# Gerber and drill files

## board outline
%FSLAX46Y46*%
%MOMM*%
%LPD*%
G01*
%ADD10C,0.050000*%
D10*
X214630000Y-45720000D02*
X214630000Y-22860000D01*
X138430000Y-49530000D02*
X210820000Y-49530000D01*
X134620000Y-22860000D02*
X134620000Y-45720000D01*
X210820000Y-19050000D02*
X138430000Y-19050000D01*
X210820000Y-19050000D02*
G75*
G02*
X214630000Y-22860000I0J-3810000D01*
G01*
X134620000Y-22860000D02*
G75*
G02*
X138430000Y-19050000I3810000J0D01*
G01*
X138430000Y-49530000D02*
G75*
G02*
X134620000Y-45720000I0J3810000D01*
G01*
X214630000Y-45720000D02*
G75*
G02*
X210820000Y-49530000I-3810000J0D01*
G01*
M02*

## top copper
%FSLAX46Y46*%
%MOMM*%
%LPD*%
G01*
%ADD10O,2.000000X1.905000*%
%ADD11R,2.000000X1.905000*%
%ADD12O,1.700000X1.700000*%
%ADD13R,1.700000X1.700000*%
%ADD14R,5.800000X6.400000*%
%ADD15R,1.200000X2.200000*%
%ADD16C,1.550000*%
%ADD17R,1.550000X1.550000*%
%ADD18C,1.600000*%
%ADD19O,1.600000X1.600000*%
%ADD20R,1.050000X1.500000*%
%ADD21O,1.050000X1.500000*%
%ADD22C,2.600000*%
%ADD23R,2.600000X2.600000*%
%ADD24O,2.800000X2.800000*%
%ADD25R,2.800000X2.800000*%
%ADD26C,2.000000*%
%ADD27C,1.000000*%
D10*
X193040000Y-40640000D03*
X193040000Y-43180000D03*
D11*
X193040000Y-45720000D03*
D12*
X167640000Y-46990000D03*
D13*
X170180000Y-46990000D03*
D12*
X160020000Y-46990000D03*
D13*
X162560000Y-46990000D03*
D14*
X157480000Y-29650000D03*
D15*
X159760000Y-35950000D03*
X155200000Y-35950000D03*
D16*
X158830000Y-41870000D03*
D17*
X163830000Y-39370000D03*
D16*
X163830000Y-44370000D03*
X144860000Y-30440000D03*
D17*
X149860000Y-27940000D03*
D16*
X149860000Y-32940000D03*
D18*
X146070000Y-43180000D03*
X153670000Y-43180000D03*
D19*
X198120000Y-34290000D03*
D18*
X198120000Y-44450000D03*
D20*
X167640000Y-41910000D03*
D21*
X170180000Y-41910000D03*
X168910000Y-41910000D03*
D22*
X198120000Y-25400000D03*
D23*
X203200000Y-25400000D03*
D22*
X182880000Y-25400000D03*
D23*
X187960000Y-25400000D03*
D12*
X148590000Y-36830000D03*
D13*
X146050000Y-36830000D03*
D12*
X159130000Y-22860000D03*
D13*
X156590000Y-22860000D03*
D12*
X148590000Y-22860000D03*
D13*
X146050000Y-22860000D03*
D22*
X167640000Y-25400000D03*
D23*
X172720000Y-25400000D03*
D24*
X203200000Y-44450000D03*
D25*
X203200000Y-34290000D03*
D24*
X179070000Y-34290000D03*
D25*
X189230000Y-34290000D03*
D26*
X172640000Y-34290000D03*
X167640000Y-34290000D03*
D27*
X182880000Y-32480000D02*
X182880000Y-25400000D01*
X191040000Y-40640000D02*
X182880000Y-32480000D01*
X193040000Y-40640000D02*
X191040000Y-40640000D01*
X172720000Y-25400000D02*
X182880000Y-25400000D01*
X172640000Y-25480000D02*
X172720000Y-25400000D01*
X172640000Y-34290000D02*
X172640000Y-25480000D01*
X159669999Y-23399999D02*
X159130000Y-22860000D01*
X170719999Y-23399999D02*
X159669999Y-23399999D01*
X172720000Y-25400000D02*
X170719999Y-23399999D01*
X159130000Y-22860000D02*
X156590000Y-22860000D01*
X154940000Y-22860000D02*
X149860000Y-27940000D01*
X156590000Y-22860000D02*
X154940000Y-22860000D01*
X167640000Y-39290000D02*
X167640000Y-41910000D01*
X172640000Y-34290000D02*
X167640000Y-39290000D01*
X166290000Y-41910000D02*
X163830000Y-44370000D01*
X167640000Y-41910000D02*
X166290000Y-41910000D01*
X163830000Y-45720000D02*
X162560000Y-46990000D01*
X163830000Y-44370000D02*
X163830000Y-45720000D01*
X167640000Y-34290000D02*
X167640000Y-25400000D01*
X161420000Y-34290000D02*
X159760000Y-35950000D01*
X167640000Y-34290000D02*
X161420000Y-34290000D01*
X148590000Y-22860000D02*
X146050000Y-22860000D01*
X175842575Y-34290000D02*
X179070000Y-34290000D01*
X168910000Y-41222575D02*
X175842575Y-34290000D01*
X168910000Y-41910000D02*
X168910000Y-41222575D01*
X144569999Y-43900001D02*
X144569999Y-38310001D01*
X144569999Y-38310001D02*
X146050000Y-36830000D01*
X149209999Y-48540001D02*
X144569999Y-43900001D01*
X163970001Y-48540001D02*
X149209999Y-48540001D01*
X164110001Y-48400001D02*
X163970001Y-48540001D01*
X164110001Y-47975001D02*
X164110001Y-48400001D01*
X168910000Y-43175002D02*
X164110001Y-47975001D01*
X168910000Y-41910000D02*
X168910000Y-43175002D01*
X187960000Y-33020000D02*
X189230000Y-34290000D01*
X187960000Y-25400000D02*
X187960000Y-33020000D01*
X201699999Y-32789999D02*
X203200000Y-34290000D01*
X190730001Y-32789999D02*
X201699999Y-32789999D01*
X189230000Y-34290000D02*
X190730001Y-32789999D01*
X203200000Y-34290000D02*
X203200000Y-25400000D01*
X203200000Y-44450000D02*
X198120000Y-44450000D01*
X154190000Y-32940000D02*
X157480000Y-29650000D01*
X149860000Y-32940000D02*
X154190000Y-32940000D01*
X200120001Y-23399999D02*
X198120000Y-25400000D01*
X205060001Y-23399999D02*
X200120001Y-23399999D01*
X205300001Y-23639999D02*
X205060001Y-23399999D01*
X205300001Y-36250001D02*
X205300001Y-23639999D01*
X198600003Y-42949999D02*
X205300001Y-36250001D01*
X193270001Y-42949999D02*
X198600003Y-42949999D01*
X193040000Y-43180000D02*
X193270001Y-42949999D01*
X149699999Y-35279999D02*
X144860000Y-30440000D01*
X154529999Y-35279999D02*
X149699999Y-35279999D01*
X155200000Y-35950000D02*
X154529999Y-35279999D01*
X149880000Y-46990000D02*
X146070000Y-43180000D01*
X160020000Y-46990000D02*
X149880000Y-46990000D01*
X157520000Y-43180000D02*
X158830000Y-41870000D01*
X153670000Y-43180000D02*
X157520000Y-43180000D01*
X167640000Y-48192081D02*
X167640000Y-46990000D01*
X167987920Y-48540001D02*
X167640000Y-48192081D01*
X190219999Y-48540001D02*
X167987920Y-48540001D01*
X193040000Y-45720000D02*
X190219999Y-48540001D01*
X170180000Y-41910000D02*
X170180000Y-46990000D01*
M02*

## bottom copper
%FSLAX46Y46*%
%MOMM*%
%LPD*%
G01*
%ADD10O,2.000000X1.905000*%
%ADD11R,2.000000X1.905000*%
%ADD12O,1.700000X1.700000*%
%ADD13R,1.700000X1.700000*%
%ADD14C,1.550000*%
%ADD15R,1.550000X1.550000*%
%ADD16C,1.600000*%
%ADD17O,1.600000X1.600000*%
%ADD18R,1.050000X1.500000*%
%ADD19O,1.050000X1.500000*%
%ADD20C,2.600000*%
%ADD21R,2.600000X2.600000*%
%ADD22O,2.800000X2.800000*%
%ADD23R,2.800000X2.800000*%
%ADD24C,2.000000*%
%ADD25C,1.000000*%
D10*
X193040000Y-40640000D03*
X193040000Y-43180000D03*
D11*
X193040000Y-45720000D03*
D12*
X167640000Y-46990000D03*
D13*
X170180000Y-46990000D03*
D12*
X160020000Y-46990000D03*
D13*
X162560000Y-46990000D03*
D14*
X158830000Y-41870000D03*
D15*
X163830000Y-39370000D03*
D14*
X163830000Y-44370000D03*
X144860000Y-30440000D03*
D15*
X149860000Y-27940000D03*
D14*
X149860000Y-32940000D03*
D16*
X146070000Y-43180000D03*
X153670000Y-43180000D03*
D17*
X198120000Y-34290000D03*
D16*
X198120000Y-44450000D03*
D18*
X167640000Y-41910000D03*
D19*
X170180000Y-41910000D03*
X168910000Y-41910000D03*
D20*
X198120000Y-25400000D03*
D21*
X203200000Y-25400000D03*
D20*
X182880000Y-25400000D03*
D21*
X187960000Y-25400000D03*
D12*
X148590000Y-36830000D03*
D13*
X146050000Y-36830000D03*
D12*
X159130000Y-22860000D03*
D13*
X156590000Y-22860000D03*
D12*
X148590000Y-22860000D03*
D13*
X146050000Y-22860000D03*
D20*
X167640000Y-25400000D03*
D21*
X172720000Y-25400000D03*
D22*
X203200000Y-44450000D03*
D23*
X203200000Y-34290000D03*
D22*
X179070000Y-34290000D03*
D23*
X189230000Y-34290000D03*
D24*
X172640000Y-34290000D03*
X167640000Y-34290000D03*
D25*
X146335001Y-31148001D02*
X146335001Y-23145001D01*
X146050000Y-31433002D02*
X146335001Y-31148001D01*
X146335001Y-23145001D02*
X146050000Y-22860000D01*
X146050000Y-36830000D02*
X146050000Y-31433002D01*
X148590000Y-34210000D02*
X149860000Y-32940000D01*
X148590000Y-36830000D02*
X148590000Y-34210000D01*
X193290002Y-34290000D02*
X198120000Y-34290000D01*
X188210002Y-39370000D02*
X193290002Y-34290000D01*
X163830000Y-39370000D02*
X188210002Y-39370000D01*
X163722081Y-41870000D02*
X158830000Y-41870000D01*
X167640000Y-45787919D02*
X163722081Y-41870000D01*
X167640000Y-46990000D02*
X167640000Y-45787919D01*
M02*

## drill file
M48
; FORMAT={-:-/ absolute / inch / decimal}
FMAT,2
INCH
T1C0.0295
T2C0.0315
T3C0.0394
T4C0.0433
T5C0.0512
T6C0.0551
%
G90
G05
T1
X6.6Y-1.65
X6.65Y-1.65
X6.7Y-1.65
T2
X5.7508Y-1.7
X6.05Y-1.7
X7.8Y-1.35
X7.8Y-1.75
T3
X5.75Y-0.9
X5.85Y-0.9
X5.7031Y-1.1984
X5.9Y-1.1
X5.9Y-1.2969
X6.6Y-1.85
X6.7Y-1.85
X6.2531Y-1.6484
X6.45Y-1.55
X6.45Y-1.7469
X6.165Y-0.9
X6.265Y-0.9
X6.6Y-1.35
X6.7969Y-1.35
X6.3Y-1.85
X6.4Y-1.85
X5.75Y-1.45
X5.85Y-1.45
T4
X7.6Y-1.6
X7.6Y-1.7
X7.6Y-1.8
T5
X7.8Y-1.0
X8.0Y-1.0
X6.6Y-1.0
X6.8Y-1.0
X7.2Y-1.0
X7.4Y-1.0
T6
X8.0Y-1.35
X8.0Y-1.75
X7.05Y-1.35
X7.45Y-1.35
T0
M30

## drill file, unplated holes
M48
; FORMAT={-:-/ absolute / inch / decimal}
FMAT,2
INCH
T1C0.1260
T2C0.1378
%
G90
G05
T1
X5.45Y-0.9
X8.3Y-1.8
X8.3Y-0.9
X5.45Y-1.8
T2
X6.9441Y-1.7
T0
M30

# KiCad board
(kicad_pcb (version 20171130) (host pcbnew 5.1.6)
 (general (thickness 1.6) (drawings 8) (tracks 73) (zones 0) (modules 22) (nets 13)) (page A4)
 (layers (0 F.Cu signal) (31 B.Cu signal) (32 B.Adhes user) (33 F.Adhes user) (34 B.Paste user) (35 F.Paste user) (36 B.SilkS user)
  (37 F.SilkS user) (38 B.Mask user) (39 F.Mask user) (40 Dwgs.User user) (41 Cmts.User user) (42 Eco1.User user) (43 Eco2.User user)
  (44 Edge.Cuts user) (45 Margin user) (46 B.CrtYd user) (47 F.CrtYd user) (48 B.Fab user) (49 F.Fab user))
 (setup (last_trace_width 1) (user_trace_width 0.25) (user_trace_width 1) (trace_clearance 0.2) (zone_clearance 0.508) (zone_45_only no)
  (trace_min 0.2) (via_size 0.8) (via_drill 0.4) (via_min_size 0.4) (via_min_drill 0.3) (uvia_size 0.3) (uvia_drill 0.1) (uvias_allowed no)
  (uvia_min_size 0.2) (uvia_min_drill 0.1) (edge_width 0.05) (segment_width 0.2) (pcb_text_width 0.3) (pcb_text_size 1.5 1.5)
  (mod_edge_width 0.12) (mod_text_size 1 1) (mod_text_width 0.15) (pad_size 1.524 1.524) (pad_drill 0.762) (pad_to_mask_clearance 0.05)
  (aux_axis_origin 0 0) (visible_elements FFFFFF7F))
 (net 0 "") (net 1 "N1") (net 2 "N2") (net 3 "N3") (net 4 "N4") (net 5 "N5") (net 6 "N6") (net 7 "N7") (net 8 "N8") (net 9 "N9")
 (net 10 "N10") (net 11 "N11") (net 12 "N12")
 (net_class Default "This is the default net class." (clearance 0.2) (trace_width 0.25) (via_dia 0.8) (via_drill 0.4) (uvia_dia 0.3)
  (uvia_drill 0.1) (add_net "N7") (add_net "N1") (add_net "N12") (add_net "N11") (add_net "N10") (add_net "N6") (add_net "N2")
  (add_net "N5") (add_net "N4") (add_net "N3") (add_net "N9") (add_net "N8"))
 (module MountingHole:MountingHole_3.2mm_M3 (layer F.Cu) (at 210.82 22.86)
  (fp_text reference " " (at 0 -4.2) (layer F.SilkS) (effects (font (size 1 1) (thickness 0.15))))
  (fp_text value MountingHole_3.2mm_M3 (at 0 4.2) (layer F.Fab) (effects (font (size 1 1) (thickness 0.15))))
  (pad 1 np_thru_hole circle (at 0 0) (size 3.2 3.2) (drill 3.2) (layers *.Cu *.Mask)))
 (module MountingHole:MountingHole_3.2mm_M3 (layer F.Cu) (at 210.82 45.72)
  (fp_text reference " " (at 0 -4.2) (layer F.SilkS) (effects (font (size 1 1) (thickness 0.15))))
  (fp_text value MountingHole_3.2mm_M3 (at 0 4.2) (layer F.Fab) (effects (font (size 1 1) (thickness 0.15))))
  (pad 1 np_thru_hole circle (at 0 0) (size 3.2 3.2) (drill 3.2) (layers *.Cu *.Mask)))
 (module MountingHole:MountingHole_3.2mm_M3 (layer F.Cu) (at 138.43 45.72)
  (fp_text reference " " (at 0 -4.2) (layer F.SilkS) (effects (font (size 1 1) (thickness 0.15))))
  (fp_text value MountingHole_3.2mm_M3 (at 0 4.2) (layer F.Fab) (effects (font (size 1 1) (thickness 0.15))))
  (pad 1 np_thru_hole circle (at 0 0) (size 3.2 3.2) (drill 3.2) (layers *.Cu *.Mask)))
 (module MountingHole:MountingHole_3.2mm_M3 (layer F.Cu) (at 138.43 22.86)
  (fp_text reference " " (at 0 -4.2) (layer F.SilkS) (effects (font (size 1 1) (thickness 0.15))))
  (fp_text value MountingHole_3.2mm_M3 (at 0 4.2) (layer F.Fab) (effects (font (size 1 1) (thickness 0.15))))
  (pad 1 np_thru_hole circle (at 0 0) (size 3.2 3.2) (drill 3.2) (layers *.Cu *.Mask)))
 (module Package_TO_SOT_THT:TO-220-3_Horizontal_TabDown (layer F.Cu) (at 193.04 45.72 90)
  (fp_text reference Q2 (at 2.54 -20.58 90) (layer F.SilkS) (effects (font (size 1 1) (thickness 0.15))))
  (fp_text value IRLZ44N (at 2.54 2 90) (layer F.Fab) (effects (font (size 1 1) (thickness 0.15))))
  (pad 3 thru_hole oval (at 5.08 0 90) (size 1.905 2) (drill 1.1) (layers *.Cu *.Mask) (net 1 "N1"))
  (pad 2 thru_hole oval (at 2.54 0 90) (size 1.905 2) (drill 1.1) (layers *.Cu *.Mask) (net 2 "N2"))
  (pad 1 thru_hole rect (at 0 0 90) (size 1.905 2) (drill 1.1) (layers *.Cu *.Mask) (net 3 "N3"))
  (pad "" np_thru_hole oval (at 2.54 -16.66 90) (size 3.5 3.5) (drill 3.5) (layers *.Cu *.Mask)))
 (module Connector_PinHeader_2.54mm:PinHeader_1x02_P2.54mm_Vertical (layer F.Cu) (at 170.18 46.99 270)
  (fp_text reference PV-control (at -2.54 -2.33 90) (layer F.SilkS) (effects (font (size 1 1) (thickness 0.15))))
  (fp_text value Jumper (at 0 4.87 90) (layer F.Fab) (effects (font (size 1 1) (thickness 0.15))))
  (pad 2 thru_hole oval (at 0 2.54 270) (size 1.7 1.7) (drill 1) (layers *.Cu *.Mask) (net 3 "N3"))
  (pad 1 thru_hole rect (at 0 0 270) (size 1.7 1.7) (drill 1) (layers *.Cu *.Mask) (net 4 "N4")))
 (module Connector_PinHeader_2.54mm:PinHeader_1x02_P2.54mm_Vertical (layer F.Cu) (at 162.56 46.99 270)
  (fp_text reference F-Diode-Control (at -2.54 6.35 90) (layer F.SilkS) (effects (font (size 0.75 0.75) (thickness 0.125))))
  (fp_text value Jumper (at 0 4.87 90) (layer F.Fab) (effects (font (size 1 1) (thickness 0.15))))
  (pad 2 thru_hole oval (at 0 2.54 270) (size 1.7 1.7) (drill 1) (layers *.Cu *.Mask) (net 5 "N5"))
  (pad 1 thru_hole rect (at 0 0 270) (size 1.7 1.7) (drill 1) (layers *.Cu *.Mask) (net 1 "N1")))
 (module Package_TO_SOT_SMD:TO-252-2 (layer F.Cu) (at 157.48 31.75 90)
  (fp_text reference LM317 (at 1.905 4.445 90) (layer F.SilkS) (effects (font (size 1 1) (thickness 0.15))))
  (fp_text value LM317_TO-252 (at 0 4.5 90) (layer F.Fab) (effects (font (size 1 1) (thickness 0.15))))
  (pad "" smd rect (at 0.425 1.525 90) (size 3.05 2.75) (layers F.Paste))
  (pad "" smd rect (at 3.775 -1.525 90) (size 3.05 2.75) (layers F.Paste))
  (pad "" smd rect (at 0.425 -1.525 90) (size 3.05 2.75) (layers F.Paste))
  (pad "" smd rect (at 3.775 1.525 90) (size 3.05 2.75) (layers F.Paste))
  (pad 2 smd rect (at 2.1 0 90) (size 6.4 5.8) (layers F.Cu F.Mask) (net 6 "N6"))
  (pad 3 smd rect (at -4.2 2.28 90) (size 2.2 1.2) (layers F.Cu F.Paste F.Mask) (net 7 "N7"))
  (pad 1 smd rect (at -4.2 -2.28 90) (size 2.2 1.2) (layers F.Cu F.Paste F.Mask) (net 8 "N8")))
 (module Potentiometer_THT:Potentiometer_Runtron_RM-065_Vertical (layer F.Cu) (at 163.83 39.37 270)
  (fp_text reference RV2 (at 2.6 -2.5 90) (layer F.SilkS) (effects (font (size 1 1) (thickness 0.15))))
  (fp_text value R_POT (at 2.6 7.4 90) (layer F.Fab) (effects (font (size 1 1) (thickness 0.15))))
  (pad 2 thru_hole circle (at 2.5 5 270) (size 1.55 1.55) (drill 1) (layers *.Cu *.Mask) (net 3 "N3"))
  (pad 1 thru_hole rect (at 0 0 270) (size 1.55 1.55) (drill 1) (layers *.Cu *.Mask) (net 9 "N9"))
  (pad 3 thru_hole circle (at 5 0 270) (size 1.55 1.55) (drill 1) (layers *.Cu *.Mask) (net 1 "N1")))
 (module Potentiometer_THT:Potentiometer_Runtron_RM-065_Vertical (layer F.Cu) (at 149.86 27.94 270)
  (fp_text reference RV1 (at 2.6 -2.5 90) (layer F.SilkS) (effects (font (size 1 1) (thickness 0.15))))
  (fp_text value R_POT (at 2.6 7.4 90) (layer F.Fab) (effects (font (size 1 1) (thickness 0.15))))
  (pad 2 thru_hole circle (at 2.5 5 270) (size 1.55 1.55) (drill 1) (layers *.Cu *.Mask) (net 8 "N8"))
  (pad 1 thru_hole rect (at 0 0 270) (size 1.55 1.55) (drill 1) (layers *.Cu *.Mask) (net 1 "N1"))
  (pad 3 thru_hole circle (at 5 0 270) (size 1.55 1.55) (drill 1) (layers *.Cu *.Mask) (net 6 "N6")))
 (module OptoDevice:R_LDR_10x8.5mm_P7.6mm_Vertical (layer F.Cu) (at 153.67 43.18 180)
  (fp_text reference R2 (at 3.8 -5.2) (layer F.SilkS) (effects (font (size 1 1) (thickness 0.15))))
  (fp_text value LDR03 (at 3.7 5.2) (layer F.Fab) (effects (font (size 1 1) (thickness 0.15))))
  (pad 2 thru_hole circle (at 7.6 0 180) (size 1.6 1.6) (drill 0.8) (layers *.Cu *.Mask) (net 5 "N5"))
  (pad 1 thru_hole circle (at 0 0 180) (size 1.6 1.6) (drill 0.8) (layers *.Cu *.Mask) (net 3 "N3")))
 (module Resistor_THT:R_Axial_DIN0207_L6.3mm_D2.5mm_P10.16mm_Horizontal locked (layer F.Cu) (at 198.12 44.45 90)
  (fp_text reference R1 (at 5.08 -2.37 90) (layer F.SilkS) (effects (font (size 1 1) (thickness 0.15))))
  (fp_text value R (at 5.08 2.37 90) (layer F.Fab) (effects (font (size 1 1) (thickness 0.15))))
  (pad 2 thru_hole oval (at 10.16 0 90) (size 1.6 1.6) (drill 0.8) (layers *.Cu *.Mask) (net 9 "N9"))
  (pad 1 thru_hole circle (at 0 0 90) (size 1.6 1.6) (drill 0.8) (layers *.Cu *.Mask) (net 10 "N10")))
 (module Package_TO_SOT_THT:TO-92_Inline (layer F.Cu) (at 167.64 41.91)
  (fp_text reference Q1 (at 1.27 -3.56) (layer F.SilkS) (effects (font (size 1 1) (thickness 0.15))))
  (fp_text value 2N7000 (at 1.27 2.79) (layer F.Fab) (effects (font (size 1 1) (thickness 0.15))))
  (pad 1 thru_hole rect (at 0 0) (size 1.05 1.5) (drill 0.75) (layers *.Cu *.Mask) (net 1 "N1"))
  (pad 3 thru_hole oval (at 2.54 0) (size 1.05 1.5) (drill 0.75) (layers *.Cu *.Mask) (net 4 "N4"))
  (pad 2 thru_hole oval (at 1.27 0) (size 1.05 1.5) (drill 0.75) (layers *.Cu *.Mask) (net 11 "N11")))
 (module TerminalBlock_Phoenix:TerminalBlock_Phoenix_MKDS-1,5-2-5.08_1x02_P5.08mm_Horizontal (layer F.Cu) (at 203.2 25.4 180)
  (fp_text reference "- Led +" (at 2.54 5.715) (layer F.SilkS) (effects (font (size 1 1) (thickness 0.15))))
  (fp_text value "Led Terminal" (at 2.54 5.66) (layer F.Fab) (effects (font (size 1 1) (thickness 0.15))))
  (pad 2 thru_hole circle (at 5.08 0 180) (size 2.6 2.6) (drill 1.3) (layers *.Cu *.Mask) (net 2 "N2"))
  (pad 1 thru_hole rect (at 0 0 180) (size 2.6 2.6) (drill 1.3) (layers *.Cu *.Mask) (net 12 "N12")))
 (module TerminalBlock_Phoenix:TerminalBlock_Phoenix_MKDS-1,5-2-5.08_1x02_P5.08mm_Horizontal (layer F.Cu) (at 187.96 25.4 180)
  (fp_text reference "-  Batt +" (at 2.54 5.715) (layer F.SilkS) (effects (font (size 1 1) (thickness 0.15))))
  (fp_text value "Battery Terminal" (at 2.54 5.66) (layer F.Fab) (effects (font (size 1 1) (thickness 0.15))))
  (pad 2 thru_hole circle (at 5.08 0 180) (size 2.6 2.6) (drill 1.3) (layers *.Cu *.Mask) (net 1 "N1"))
  (pad 1 thru_hole rect (at 0 0 180) (size 2.6 2.6) (drill 1.3) (layers *.Cu *.Mask) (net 12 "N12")))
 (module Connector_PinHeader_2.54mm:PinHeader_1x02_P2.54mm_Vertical (layer F.Cu) (at 146.05 36.83 90)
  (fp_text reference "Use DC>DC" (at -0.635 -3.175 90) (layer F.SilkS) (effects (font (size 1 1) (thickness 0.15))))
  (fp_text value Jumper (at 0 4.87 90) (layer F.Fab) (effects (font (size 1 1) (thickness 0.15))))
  (pad 2 thru_hole oval (at 0 2.54 90) (size 1.7 1.7) (drill 1) (layers *.Cu *.Mask) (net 6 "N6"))
  (pad 1 thru_hole rect (at 0 0 90) (size 1.7 1.7) (drill 1) (layers *.Cu *.Mask) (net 11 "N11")))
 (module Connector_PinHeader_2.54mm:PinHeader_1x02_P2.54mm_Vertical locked (layer F.Cu) (at 156.59 22.86 90)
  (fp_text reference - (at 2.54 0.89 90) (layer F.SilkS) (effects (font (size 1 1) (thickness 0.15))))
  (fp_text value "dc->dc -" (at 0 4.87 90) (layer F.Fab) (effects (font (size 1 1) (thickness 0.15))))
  (pad 2 thru_hole oval (at 0 2.54 90) (size 1.7 1.7) (drill 1) (layers *.Cu *.Mask) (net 1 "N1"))
  (pad 1 thru_hole rect (at 0 0 90) (size 1.7 1.7) (drill 1) (layers *.Cu *.Mask) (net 1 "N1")))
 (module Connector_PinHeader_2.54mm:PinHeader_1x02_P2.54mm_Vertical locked (layer F.Cu) (at 146.05 22.86 90)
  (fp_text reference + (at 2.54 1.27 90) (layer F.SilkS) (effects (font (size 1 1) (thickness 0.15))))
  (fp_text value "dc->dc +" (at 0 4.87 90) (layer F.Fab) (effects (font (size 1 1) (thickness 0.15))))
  (pad 2 thru_hole oval (at 0 2.54 90) (size 1.7 1.7) (drill 1) (layers *.Cu *.Mask) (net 11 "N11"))
  (pad 1 thru_hole rect (at 0 0 90) (size 1.7 1.7) (drill 1) (layers *.Cu *.Mask) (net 11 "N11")))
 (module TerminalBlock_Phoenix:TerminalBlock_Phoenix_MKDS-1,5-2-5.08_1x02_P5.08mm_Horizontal (layer F.Cu) (at 172.72 25.4 180)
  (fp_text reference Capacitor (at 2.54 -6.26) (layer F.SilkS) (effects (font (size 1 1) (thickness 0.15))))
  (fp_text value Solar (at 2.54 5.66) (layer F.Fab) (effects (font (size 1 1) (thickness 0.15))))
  (pad 2 thru_hole circle (at 5.08 0 180) (size 2.6 2.6) (drill 1.3) (layers *.Cu *.Mask) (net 7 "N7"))
  (pad 1 thru_hole rect (at 0 0 180) (size 2.6 2.6) (drill 1.3) (layers *.Cu *.Mask) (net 1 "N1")))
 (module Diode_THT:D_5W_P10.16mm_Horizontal (layer F.Cu) (at 203.2 34.29 270)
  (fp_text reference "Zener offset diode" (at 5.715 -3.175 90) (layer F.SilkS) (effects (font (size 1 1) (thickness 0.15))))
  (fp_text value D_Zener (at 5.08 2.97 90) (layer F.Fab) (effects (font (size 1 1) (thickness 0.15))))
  (pad 2 thru_hole oval (at 10.16 0 270) (size 2.8 2.8) (drill 1.4) (layers *.Cu *.Mask) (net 10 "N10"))
  (pad 1 thru_hole rect (at 0 0 270) (size 2.8 2.8) (drill 1.4) (layers *.Cu *.Mask) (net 12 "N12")))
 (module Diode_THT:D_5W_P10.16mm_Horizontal (layer F.Cu) (at 189.23 34.29 180)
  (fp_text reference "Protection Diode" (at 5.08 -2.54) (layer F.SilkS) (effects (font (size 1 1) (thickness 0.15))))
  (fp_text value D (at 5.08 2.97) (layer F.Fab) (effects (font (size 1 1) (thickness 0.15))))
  (pad 2 thru_hole oval (at 10.16 0 180) (size 2.8 2.8) (drill 1.4) (layers *.Cu *.Mask) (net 11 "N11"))
  (pad 1 thru_hole rect (at 0 0 180) (size 2.8 2.8) (drill 1.4) (layers *.Cu *.Mask) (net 12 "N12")))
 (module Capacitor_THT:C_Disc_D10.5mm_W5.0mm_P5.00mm (layer F.Cu) (at 167.64 34.29)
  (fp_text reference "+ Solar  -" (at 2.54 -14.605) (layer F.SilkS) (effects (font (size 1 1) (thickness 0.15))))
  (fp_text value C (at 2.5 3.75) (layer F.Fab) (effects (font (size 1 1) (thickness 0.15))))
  (pad 2 thru_hole circle (at 5 0) (size 2 2) (drill 1) (layers *.Cu *.Mask) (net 1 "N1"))
  (pad 1 thru_hole circle (at 0 0) (size 2 2) (drill 1) (layers *.Cu *.Mask) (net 7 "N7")))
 (gr_line (start 214.63 45.72) (end 214.63 22.86) (layer Edge.Cuts) (width 0.05))
 (gr_line (start 138.43 49.53) (end 210.82 49.53) (layer Edge.Cuts) (width 0.05))
 (gr_line (start 134.62 22.86) (end 134.62 45.72) (layer Edge.Cuts) (width 0.05))
 (gr_line (start 210.82 19.05) (end 138.43 19.05) (layer Edge.Cuts) (width 0.05))
 (gr_arc (start 210.82 22.86) (end 214.63 22.86) (angle -90) (layer Edge.Cuts) (width 0.05))
 (gr_arc (start 138.43 22.86) (end 138.43 19.05) (angle -90) (layer Edge.Cuts) (width 0.05))
 (gr_arc (start 138.43 45.72) (end 134.62 45.72) (angle -90) (layer Edge.Cuts) (width 0.05))
 (gr_arc (start 210.82 45.72) (end 210.82 49.53) (angle -90) (layer Edge.Cuts) (width 0.05))
 (segment (start 182.88 32.48) (end 182.88 25.4) (width 1) (layer F.Cu) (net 1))
 (segment (start 191.04 40.64) (end 182.88 32.48) (width 1) (layer F.Cu) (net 1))
 (segment (start 193.04 40.64) (end 191.04 40.64) (width 1) (layer F.Cu) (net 1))
 (segment (start 172.72 25.4) (end 182.88 25.4) (width 1) (layer F.Cu) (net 1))
 (segment (start 172.64 25.48) (end 172.72 25.4) (width 1) (layer F.Cu) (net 1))
 (segment (start 172.64 34.29) (end 172.64 25.48) (width 1) (layer F.Cu) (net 1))
 (segment (start 159.669999 23.399999) (end 159.13 22.86) (width 1) (layer F.Cu) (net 1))
 (segment (start 170.719999 23.399999) (end 159.669999 23.399999) (width 1) (layer F.Cu) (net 1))
 (segment (start 172.72 25.4) (end 170.719999 23.399999) (width 1) (layer F.Cu) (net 1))
 (segment (start 159.13 22.86) (end 156.59 22.86) (width 1) (layer F.Cu) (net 1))
 (segment (start 154.94 22.86) (end 149.86 27.94) (width 1) (layer F.Cu) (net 1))
 (segment (start 156.59 22.86) (end 154.94 22.86) (width 1) (layer F.Cu) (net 1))
 (segment (start 167.64 39.29) (end 167.64 41.91) (width 1) (layer F.Cu) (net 1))
 (segment (start 172.64 34.29) (end 167.64 39.29) (width 1) (layer F.Cu) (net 1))
 (segment (start 166.29 41.91) (end 163.83 44.37) (width 1) (layer F.Cu) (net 1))
 (segment (start 167.64 41.91) (end 166.29 41.91) (width 1) (layer F.Cu) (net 1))
 (segment (start 163.83 45.72) (end 162.56 46.99) (width 1) (layer F.Cu) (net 1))
 (segment (start 163.83 44.37) (end 163.83 45.72) (width 1) (layer F.Cu) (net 1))
 (segment (start 167.64 34.29) (end 167.64 25.4) (width 1) (layer F.Cu) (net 7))
 (segment (start 161.42 34.29) (end 159.76 35.95) (width 1) (layer F.Cu) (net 7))
 (segment (start 167.64 34.29) (end 161.42 34.29) (width 1) (layer F.Cu) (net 7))
 (segment (start 148.59 22.86) (end 146.05 22.86) (width 1) (layer F.Cu) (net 11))
 (segment (start 175.842575 34.29) (end 179.07 34.29) (width 1) (layer F.Cu) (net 11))
 (segment (start 168.91 41.222575) (end 175.842575 34.29) (width 1) (layer F.Cu) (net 11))
 (segment (start 168.91 41.91) (end 168.91 41.222575) (width 1) (layer F.Cu) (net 11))
 (segment (start 144.569999 43.900001) (end 144.569999 38.310001) (width 1) (layer F.Cu) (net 11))
 (segment (start 144.569999 38.310001) (end 146.05 36.83) (width 1) (layer F.Cu) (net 11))
 (segment (start 149.209999 48.540001) (end 144.569999 43.900001) (width 1) (layer F.Cu) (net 11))
 (segment (start 163.970001 48.540001) (end 149.209999 48.540001) (width 1) (layer F.Cu) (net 11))
 (segment (start 164.110001 48.400001) (end 163.970001 48.540001) (width 1) (layer F.Cu) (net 11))
 (segment (start 164.110001 47.975001) (end 164.110001 48.400001) (width 1) (layer F.Cu) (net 11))
 (segment (start 168.91 43.175002) (end 164.110001 47.975001) (width 1) (layer F.Cu) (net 11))
 (segment (start 168.91 41.91) (end 168.91 43.175002) (width 1) (layer F.Cu) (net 11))
 (segment (start 146.335001 31.148001) (end 146.335001 23.145001) (width 1) (layer B.Cu) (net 11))
 (segment (start 146.05 31.433002) (end 146.335001 31.148001) (width 1) (layer B.Cu) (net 11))
 (segment (start 146.335001 23.145001) (end 146.05 22.86) (width 1) (layer B.Cu) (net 11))
 (segment (start 146.05 36.83) (end 146.05 31.433002) (width 1) (layer B.Cu) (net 11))
 (segment (start 187.96 33.02) (end 189.23 34.29) (width 1) (layer F.Cu) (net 12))
 (segment (start 187.96 25.4) (end 187.96 33.02) (width 1) (layer F.Cu) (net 12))
 (segment (start 201.699999 32.789999) (end 203.2 34.29) (width 1) (layer F.Cu) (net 12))
 (segment (start 190.730001 32.789999) (end 201.699999 32.789999) (width 1) (layer F.Cu) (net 12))
 (segment (start 189.23 34.29) (end 190.730001 32.789999) (width 1) (layer F.Cu) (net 12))
 (segment (start 203.2 34.29) (end 203.2 25.4) (width 1) (layer F.Cu) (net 12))
 (segment (start 203.2 44.45) (end 198.12 44.45) (width 1) (layer F.Cu) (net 10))
 (segment (start 148.59 34.21) (end 149.86 32.94) (width 1) (layer B.Cu) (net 6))
 (segment (start 148.59 36.83) (end 148.59 34.21) (width 1) (layer B.Cu) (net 6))
 (segment (start 154.19 32.94) (end 157.48 29.65) (width 1) (layer F.Cu) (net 6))
 (segment (start 149.86 32.94) (end 154.19 32.94) (width 1) (layer F.Cu) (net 6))
 (segment (start 200.120001 23.399999) (end 198.12 25.4) (width 1) (layer F.Cu) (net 2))
 (segment (start 205.060001 23.399999) (end 200.120001 23.399999) (width 1) (layer F.Cu) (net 2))
 (segment (start 205.300001 23.639999) (end 205.060001 23.399999) (width 1) (layer F.Cu) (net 2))
 (segment (start 205.300001 36.250001) (end 205.300001 23.639999) (width 1) (layer F.Cu) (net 2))
 (segment (start 198.600003 42.949999) (end 205.300001 36.250001) (width 1) (layer F.Cu) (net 2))
 (segment (start 193.270001 42.949999) (end 198.600003 42.949999) (width 1) (layer F.Cu) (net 2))
 (segment (start 193.04 43.18) (end 193.270001 42.949999) (width 1) (layer F.Cu) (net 2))
 (segment (start 193.290002 34.29) (end 198.12 34.29) (width 1) (layer B.Cu) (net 9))
 (segment (start 188.210002 39.37) (end 193.290002 34.29) (width 1) (layer B.Cu) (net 9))
 (segment (start 163.83 39.37) (end 188.210002 39.37) (width 1) (layer B.Cu) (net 9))
 (segment (start 149.699999 35.279999) (end 144.86 30.44) (width 1) (layer F.Cu) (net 8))
 (segment (start 154.529999 35.279999) (end 149.699999 35.279999) (width 1) (layer F.Cu) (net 8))
 (segment (start 155.2 35.95) (end 154.529999 35.279999) (width 1) (layer F.Cu) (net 8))
 (segment (start 149.88 46.99) (end 146.07 43.18) (width 1) (layer F.Cu) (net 5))
 (segment (start 160.02 46.99) (end 149.88 46.99) (width 1) (layer F.Cu) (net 5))
 (segment (start 157.52 43.18) (end 158.83 41.87) (width 1) (layer F.Cu) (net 3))
 (segment (start 153.67 43.18) (end 157.52 43.18) (width 1) (layer F.Cu) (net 3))
 (segment (start 167.64 48.192081) (end 167.64 46.99) (width 1) (layer F.Cu) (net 3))
 (segment (start 167.98792 48.540001) (end 167.64 48.192081) (width 1) (layer F.Cu) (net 3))
 (segment (start 190.219999 48.540001) (end 167.98792 48.540001) (width 1) (layer F.Cu) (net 3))
 (segment (start 193.04 45.72) (end 190.219999 48.540001) (width 1) (layer F.Cu) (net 3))
 (segment (start 163.722081 41.87) (end 158.83 41.87) (width 1) (layer B.Cu) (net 3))
 (segment (start 167.64 45.787919) (end 163.722081 41.87) (width 1) (layer B.Cu) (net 3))
 (segment (start 167.64 46.99) (end 167.64 45.787919) (width 1) (layer B.Cu) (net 3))
 (segment (start 170.18 41.91) (end 170.18 46.99) (width 1) (layer F.Cu) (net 4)))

